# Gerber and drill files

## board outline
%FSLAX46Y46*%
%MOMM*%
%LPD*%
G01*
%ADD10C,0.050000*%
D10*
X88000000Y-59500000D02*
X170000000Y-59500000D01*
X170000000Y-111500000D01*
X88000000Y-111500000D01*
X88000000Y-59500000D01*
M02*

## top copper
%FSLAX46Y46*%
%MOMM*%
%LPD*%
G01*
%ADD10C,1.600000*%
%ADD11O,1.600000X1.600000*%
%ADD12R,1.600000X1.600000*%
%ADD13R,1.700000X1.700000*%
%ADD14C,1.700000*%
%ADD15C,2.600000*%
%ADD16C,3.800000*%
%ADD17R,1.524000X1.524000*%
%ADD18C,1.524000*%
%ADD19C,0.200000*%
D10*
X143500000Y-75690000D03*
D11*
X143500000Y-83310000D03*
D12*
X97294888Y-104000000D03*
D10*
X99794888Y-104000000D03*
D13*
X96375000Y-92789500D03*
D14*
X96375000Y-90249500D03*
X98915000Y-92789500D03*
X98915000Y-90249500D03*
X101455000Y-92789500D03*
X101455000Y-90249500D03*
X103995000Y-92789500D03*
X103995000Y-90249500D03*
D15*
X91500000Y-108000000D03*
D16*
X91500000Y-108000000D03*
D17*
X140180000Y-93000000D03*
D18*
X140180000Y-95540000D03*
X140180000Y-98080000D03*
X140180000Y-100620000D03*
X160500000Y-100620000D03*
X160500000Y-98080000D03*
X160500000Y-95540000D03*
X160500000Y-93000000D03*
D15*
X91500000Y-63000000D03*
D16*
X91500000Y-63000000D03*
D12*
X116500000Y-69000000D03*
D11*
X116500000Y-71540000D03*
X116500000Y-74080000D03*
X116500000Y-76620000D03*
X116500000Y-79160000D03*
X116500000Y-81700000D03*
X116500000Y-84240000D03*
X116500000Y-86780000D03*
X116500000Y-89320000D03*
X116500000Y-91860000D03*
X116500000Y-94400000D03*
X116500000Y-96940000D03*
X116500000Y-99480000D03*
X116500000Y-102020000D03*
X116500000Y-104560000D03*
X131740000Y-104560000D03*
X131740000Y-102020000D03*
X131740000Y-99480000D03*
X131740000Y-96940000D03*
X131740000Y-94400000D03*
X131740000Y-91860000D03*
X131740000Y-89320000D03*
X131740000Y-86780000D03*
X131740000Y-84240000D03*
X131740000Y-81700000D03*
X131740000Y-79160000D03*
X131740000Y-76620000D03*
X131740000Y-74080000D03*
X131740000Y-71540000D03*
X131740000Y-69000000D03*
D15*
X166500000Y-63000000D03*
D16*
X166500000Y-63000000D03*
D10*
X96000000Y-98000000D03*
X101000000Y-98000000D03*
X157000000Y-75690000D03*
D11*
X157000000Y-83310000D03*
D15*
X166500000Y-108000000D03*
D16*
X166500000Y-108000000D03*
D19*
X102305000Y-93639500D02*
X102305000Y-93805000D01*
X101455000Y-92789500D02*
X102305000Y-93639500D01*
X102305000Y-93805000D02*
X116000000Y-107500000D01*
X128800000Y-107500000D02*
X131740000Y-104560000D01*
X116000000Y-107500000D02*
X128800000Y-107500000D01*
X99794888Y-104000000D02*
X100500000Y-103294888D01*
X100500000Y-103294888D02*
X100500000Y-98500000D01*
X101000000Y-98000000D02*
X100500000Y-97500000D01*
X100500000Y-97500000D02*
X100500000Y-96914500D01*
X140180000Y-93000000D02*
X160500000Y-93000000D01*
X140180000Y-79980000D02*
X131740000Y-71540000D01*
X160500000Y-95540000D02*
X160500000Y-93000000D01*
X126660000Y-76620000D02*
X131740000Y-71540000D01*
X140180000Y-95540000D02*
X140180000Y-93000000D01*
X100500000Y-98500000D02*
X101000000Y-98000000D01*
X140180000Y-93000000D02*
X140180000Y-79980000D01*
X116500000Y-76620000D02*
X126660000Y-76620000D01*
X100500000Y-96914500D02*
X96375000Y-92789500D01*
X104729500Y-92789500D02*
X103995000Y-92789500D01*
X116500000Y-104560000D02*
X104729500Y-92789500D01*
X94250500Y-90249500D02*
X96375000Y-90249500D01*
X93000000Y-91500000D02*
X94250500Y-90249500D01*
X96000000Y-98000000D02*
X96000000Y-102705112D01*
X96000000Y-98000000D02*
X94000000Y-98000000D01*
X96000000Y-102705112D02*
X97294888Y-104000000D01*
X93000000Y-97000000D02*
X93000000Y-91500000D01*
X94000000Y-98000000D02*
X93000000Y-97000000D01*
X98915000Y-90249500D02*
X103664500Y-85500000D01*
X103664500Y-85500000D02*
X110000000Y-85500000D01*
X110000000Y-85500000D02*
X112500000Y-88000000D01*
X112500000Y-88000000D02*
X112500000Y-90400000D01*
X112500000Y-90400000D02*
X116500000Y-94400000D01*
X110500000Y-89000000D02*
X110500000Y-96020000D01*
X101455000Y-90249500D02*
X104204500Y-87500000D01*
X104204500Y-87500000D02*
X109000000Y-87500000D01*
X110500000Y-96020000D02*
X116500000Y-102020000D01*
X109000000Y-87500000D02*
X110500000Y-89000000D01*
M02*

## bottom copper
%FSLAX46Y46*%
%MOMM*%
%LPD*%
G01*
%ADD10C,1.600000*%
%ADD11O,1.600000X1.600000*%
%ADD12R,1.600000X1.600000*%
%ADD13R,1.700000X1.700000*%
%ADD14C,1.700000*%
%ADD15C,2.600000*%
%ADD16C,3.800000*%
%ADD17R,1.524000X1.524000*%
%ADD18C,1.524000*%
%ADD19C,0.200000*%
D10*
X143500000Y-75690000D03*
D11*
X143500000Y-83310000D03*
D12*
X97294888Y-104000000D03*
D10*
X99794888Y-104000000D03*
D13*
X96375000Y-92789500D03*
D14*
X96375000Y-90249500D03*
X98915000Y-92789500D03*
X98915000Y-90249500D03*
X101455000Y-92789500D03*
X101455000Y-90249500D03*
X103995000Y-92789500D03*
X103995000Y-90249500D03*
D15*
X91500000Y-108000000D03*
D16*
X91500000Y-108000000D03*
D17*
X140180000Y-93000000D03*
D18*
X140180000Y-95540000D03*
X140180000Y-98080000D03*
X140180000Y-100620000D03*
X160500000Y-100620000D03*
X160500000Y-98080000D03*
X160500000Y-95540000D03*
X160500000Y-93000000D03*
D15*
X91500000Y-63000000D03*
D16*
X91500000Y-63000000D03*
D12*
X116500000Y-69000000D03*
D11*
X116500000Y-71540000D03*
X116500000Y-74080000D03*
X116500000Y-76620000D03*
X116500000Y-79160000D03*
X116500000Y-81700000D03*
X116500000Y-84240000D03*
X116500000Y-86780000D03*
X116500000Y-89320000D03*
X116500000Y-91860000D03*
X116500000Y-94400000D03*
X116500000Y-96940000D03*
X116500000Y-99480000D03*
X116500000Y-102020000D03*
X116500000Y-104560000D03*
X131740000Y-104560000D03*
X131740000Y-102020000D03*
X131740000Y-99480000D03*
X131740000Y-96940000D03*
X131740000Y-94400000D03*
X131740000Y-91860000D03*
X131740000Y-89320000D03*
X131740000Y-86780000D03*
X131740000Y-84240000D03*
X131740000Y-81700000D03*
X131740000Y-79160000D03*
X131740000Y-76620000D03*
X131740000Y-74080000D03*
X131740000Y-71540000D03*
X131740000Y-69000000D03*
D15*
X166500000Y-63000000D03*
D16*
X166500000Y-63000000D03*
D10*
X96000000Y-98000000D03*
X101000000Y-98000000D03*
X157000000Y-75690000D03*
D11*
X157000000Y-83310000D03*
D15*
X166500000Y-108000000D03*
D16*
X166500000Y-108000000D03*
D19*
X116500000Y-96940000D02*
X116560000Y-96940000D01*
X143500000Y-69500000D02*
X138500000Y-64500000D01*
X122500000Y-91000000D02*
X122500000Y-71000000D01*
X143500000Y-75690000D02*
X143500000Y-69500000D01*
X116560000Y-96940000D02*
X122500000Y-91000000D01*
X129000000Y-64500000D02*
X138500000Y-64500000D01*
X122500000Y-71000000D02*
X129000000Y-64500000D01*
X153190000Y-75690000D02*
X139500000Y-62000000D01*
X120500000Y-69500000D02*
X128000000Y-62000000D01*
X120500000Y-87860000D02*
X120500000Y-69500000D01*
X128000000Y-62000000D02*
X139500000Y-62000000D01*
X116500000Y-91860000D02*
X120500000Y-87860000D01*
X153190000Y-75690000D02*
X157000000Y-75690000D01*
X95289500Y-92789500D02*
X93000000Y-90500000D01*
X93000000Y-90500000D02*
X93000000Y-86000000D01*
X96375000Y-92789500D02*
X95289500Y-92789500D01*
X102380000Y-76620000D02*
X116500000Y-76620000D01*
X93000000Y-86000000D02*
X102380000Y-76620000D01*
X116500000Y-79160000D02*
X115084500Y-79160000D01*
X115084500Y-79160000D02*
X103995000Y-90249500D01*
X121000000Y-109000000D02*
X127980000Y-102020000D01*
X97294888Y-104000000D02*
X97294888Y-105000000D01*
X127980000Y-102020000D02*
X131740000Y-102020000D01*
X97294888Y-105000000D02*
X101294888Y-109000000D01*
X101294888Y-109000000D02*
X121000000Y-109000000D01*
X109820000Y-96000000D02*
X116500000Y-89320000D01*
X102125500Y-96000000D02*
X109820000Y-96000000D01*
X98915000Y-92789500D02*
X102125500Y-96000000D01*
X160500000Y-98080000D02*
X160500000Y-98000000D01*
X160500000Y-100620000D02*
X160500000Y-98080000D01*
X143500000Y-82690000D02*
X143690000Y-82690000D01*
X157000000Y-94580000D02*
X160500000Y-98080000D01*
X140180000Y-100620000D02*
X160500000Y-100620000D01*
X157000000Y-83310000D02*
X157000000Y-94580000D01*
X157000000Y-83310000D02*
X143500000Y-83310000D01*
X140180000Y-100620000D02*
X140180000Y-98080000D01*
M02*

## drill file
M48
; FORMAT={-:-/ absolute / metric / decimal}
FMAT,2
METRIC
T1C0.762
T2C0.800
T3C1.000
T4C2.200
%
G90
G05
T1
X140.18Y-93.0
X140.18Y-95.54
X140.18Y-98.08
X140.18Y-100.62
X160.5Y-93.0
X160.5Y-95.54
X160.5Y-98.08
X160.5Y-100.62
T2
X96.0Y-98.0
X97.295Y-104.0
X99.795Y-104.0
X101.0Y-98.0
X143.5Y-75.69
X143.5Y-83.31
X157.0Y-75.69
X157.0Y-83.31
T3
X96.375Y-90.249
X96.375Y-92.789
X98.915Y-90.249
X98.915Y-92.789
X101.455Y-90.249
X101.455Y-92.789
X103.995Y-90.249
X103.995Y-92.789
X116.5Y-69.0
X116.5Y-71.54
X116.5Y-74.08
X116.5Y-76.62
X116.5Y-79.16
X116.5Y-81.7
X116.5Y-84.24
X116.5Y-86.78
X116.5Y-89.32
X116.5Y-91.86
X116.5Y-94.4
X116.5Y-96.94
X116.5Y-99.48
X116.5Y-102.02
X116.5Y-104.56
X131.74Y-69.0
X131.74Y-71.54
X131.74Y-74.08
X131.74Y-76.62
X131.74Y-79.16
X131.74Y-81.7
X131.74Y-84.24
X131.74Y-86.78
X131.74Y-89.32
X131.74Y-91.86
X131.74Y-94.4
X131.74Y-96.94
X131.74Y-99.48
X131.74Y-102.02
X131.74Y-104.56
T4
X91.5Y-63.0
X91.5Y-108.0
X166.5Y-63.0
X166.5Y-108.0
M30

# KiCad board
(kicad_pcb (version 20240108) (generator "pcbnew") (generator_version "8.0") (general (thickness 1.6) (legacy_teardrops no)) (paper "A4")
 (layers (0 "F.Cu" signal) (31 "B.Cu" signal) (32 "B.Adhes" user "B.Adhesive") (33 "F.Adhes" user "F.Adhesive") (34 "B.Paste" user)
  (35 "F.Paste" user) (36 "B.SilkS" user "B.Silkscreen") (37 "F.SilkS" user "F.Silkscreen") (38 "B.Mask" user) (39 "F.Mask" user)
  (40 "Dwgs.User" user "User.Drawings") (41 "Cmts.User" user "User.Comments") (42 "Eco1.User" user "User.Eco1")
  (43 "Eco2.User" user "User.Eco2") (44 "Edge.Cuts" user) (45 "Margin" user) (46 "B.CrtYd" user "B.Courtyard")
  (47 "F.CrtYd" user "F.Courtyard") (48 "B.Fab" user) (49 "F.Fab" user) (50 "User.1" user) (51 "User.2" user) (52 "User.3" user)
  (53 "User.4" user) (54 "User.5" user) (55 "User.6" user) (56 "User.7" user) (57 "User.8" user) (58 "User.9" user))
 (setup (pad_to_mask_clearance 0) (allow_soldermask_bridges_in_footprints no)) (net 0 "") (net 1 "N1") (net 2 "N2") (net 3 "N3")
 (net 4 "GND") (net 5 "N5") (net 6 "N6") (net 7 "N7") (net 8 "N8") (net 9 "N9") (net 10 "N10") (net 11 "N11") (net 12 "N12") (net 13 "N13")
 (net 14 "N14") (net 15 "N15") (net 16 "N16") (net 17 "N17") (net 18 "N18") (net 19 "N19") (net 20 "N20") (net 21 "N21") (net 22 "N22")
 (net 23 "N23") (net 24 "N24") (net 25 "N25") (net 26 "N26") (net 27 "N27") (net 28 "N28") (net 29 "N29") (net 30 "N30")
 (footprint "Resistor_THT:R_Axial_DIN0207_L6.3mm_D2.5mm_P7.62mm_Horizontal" (layer "F.Cu") (at 143.5 75.69 -90)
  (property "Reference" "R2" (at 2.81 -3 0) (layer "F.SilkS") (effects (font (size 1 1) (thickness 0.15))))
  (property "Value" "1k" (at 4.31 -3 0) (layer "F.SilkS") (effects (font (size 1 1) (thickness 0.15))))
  (pad "1" thru_hole circle (at 0 0 270) (size 1.6 1.6) (drill 0.8) (layers "*.Cu" "*.Mask") (remove_unused_layers no) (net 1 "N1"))
  (pad "2" thru_hole oval (at 7.62 0 270) (size 1.6 1.6) (drill 0.8) (layers "*.Cu" "*.Mask") (remove_unused_layers no) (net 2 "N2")))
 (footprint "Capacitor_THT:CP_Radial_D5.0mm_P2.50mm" (layer "F.Cu") (at 97.294888 104)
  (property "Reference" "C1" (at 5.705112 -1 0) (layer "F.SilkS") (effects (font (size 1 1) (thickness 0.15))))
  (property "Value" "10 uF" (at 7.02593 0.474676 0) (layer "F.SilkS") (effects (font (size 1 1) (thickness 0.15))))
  (pad "1" thru_hole rect (at 0 0) (size 1.6 1.6) (drill 0.8) (layers "*.Cu" "*.Mask") (remove_unused_layers no) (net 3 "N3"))
  (pad "2" thru_hole circle (at 2.5 0) (size 1.6 1.6) (drill 0.8) (layers "*.Cu" "*.Mask") (remove_unused_layers no) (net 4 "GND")))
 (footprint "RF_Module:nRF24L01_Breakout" (layer "F.Cu") (at 96.375 92.7895 90)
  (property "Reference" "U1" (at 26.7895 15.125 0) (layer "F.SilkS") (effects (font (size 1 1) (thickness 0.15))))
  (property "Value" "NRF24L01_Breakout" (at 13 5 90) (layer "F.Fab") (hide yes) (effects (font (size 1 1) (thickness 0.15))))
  (pad "1" thru_hole rect (at 0 0 90) (size 1.7 1.7) (drill 1) (layers "*.Cu" "*.Mask") (remove_unused_layers no) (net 4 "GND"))
  (pad "2" thru_hole circle (at 2.54 0 90) (size 1.7 1.7) (drill 1) (layers "*.Cu" "*.Mask") (remove_unused_layers no) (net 3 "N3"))
  (pad "3" thru_hole circle (at 0 2.54 90) (size 1.7 1.7) (drill 1) (layers "*.Cu" "*.Mask") (remove_unused_layers no) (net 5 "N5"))
  (pad "4" thru_hole circle (at 2.54 2.54 90) (size 1.7 1.7) (drill 1) (layers "*.Cu" "*.Mask") (remove_unused_layers no) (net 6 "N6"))
  (pad "5" thru_hole circle (at 0 5.08 90) (size 1.7 1.7) (drill 1) (layers "*.Cu" "*.Mask") (remove_unused_layers no) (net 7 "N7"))
  (pad "6" thru_hole circle (at 2.54 5.08 90) (size 1.7 1.7) (drill 1) (layers "*.Cu" "*.Mask") (remove_unused_layers no) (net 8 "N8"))
  (pad "7" thru_hole circle (at 0 7.62 90) (size 1.7 1.7) (drill 1) (layers "*.Cu" "*.Mask") (remove_unused_layers no) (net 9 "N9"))
  (pad "8" thru_hole circle (at 2.54 7.62 90) (size 1.7 1.7) (drill 1) (layers "*.Cu" "*.Mask") (remove_unused_layers no) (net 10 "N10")))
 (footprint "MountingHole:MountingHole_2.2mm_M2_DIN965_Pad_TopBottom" (layer "F.Cu") (at 91.5 108)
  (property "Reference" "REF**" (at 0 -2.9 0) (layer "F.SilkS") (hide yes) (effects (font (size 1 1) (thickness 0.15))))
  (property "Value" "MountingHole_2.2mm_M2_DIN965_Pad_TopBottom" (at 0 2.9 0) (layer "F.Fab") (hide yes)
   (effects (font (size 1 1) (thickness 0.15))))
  (pad "1" thru_hole circle (at 0 0) (size 2.6 2.6) (drill 2.2) (layers "*.Cu" "*.Mask") (remove_unused_layers no))
  (pad "1" connect circle (at 0 0) (size 3.8 3.8) (layers "F.Cu" "F.Mask"))
  (pad "1" connect circle (at 0 0) (size 3.8 3.8) (layers "B.Cu" "B.Mask")))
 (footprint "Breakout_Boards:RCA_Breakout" (layer "F.Cu") (at 150.38 100.5)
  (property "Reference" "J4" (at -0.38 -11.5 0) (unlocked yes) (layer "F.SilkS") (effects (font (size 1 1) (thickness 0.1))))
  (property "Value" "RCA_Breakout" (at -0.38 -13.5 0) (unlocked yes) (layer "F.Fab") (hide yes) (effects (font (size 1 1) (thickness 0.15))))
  (pad "1" thru_hole rect (at -10.2 -7.5) (size 1.524 1.524) (drill 0.762) (layers "*.Cu" "*.Mask") (remove_unused_layers no) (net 4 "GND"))
  (pad "2" thru_hole circle (at -10.2 -4.96) (size 1.524 1.524) (drill 0.762) (layers "*.Cu" "*.Mask") (remove_unused_layers no)
   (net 4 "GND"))
  (pad "3" thru_hole circle (at -10.2 -2.42) (size 1.524 1.524) (drill 0.762) (layers "*.Cu" "*.Mask") (remove_unused_layers no)
   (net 2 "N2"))
  (pad "4" thru_hole circle (at -10.2 0.12) (size 1.524 1.524) (drill 0.762) (layers "*.Cu" "*.Mask") (remove_unused_layers no) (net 2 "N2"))
  (pad "5" thru_hole circle (at 10.12 0.12) (size 1.524 1.524) (drill 0.762) (layers "*.Cu" "*.Mask") (remove_unused_layers no) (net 2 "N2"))
  (pad "6" thru_hole circle (at 10.12 -2.42) (size 1.524 1.524) (drill 0.762) (layers "*.Cu" "*.Mask") (remove_unused_layers no)
   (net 2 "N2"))
  (pad "7" thru_hole circle (at 10.12 -4.96) (size 1.524 1.524) (drill 0.762) (layers "*.Cu" "*.Mask") (remove_unused_layers no)
   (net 4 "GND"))
  (pad "8" thru_hole circle (at 10.12 -7.5) (size 1.524 1.524) (drill 0.762) (layers "*.Cu" "*.Mask") (remove_unused_layers no)
   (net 4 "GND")))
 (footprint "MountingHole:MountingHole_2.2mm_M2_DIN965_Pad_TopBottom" (layer "F.Cu") (at 91.5 63)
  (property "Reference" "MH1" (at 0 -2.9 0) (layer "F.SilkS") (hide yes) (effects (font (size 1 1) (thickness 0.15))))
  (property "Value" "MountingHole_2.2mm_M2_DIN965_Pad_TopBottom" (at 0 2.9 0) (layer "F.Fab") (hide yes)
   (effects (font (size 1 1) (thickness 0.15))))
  (pad "1" thru_hole circle (at 0 0) (size 2.6 2.6) (drill 2.2) (layers "*.Cu" "*.Mask") (remove_unused_layers no))
  (pad "1" connect circle (at 0 0) (size 3.8 3.8) (layers "F.Cu" "F.Mask"))
  (pad "1" connect circle (at 0 0) (size 3.8 3.8) (layers "B.Cu" "B.Mask")))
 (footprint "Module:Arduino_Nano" (layer "F.Cu") (at 116.5 69)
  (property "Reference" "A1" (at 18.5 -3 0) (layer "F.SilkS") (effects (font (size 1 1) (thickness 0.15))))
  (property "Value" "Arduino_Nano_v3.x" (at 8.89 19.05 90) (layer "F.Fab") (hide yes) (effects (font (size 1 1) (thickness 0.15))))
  (pad "1" thru_hole rect (at 0 0) (size 1.6 1.6) (drill 1) (layers "*.Cu" "*.Mask") (remove_unused_layers no) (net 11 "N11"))
  (pad "2" thru_hole oval (at 0 2.54) (size 1.6 1.6) (drill 1) (layers "*.Cu" "*.Mask") (remove_unused_layers no) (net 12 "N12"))
  (pad "3" thru_hole oval (at 0 5.08) (size 1.6 1.6) (drill 1) (layers "*.Cu" "*.Mask") (remove_unused_layers no) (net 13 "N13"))
  (pad "4" thru_hole oval (at 0 7.62) (size 1.6 1.6) (drill 1) (layers "*.Cu" "*.Mask") (remove_unused_layers no) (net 4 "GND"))
  (pad "5" thru_hole oval (at 0 10.16) (size 1.6 1.6) (drill 1) (layers "*.Cu" "*.Mask") (remove_unused_layers no) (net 10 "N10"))
  (pad "6" thru_hole oval (at 0 12.7) (size 1.6 1.6) (drill 1) (layers "*.Cu" "*.Mask") (remove_unused_layers no) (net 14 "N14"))
  (pad "7" thru_hole oval (at 0 15.24) (size 1.6 1.6) (drill 1) (layers "*.Cu" "*.Mask") (remove_unused_layers no) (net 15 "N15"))
  (pad "8" thru_hole oval (at 0 17.78) (size 1.6 1.6) (drill 1) (layers "*.Cu" "*.Mask") (remove_unused_layers no) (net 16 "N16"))
  (pad "9" thru_hole oval (at 0 20.32) (size 1.6 1.6) (drill 1) (layers "*.Cu" "*.Mask") (remove_unused_layers no) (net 5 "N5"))
  (pad "10" thru_hole oval (at 0 22.86) (size 1.6 1.6) (drill 1) (layers "*.Cu" "*.Mask") (remove_unused_layers no) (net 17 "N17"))
  (pad "11" thru_hole oval (at 0 25.4) (size 1.6 1.6) (drill 1) (layers "*.Cu" "*.Mask") (remove_unused_layers no) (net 6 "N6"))
  (pad "12" thru_hole oval (at 0 27.94) (size 1.6 1.6) (drill 1) (layers "*.Cu" "*.Mask") (remove_unused_layers no) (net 1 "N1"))
  (pad "13" thru_hole oval (at 0 30.48) (size 1.6 1.6) (drill 1) (layers "*.Cu" "*.Mask") (remove_unused_layers no) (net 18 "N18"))
  (pad "14" thru_hole oval (at 0 33.02) (size 1.6 1.6) (drill 1) (layers "*.Cu" "*.Mask") (remove_unused_layers no) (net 8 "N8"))
  (pad "15" thru_hole oval (at 0 35.56) (size 1.6 1.6) (drill 1) (layers "*.Cu" "*.Mask") (remove_unused_layers no) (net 9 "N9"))
  (pad "16" thru_hole oval (at 15.24 35.56) (size 1.6 1.6) (drill 1) (layers "*.Cu" "*.Mask") (remove_unused_layers no) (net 7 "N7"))
  (pad "17" thru_hole oval (at 15.24 33.02) (size 1.6 1.6) (drill 1) (layers "*.Cu" "*.Mask") (remove_unused_layers no) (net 3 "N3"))
  (pad "18" thru_hole oval (at 15.24 30.48) (size 1.6 1.6) (drill 1) (layers "*.Cu" "*.Mask") (remove_unused_layers no) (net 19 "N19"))
  (pad "19" thru_hole oval (at 15.24 27.94) (size 1.6 1.6) (drill 1) (layers "*.Cu" "*.Mask") (remove_unused_layers no) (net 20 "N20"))
  (pad "20" thru_hole oval (at 15.24 25.4) (size 1.6 1.6) (drill 1) (layers "*.Cu" "*.Mask") (remove_unused_layers no) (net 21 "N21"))
  (pad "21" thru_hole oval (at 15.24 22.86) (size 1.6 1.6) (drill 1) (layers "*.Cu" "*.Mask") (remove_unused_layers no) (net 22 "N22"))
  (pad "22" thru_hole oval (at 15.24 20.32) (size 1.6 1.6) (drill 1) (layers "*.Cu" "*.Mask") (remove_unused_layers no) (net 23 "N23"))
  (pad "23" thru_hole oval (at 15.24 17.78) (size 1.6 1.6) (drill 1) (layers "*.Cu" "*.Mask") (remove_unused_layers no) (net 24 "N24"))
  (pad "24" thru_hole oval (at 15.24 15.24) (size 1.6 1.6) (drill 1) (layers "*.Cu" "*.Mask") (remove_unused_layers no) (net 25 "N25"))
  (pad "25" thru_hole oval (at 15.24 12.7) (size 1.6 1.6) (drill 1) (layers "*.Cu" "*.Mask") (remove_unused_layers no) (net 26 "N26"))
  (pad "26" thru_hole oval (at 15.24 10.16) (size 1.6 1.6) (drill 1) (layers "*.Cu" "*.Mask") (remove_unused_layers no) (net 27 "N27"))
  (pad "27" thru_hole oval (at 15.24 7.62) (size 1.6 1.6) (drill 1) (layers "*.Cu" "*.Mask") (remove_unused_layers no) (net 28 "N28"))
  (pad "28" thru_hole oval (at 15.24 5.08) (size 1.6 1.6) (drill 1) (layers "*.Cu" "*.Mask") (remove_unused_layers no) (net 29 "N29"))
  (pad "29" thru_hole oval (at 15.24 2.54) (size 1.6 1.6) (drill 1) (layers "*.Cu" "*.Mask") (remove_unused_layers no) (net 4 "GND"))
  (pad "30" thru_hole oval (at 15.24 0) (size 1.6 1.6) (drill 1) (layers "*.Cu" "*.Mask") (remove_unused_layers no) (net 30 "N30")))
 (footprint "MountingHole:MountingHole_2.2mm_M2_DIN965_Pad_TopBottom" (layer "F.Cu") (at 166.5 63)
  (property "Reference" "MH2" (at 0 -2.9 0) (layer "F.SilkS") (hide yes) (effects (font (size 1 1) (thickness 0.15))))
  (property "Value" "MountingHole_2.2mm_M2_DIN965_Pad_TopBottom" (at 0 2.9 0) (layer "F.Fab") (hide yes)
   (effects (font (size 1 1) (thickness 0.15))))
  (pad "1" thru_hole circle (at 0 0) (size 2.6 2.6) (drill 2.2) (layers "*.Cu" "*.Mask") (remove_unused_layers no))
  (pad "1" connect circle (at 0 0) (size 3.8 3.8) (layers "F.Cu" "F.Mask"))
  (pad "1" connect circle (at 0 0) (size 3.8 3.8) (layers "B.Cu" "B.Mask")))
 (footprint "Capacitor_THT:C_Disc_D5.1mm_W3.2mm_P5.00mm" (layer "F.Cu") (at 96 98)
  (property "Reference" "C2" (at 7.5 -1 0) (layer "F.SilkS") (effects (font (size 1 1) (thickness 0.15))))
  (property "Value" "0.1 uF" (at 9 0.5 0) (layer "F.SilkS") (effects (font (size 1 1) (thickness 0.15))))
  (pad "1" thru_hole circle (at 0 0) (size 1.6 1.6) (drill 0.8) (layers "*.Cu" "*.Mask") (remove_unused_layers no) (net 3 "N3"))
  (pad "2" thru_hole circle (at 5 0) (size 1.6 1.6) (drill 0.8) (layers "*.Cu" "*.Mask") (remove_unused_layers no) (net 4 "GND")))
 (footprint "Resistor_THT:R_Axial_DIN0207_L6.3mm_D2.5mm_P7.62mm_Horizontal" (layer "F.Cu") (at 157 75.69 -90)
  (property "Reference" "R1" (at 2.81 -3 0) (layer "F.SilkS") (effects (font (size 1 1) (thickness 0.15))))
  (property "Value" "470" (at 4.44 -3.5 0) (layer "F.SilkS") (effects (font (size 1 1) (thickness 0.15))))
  (pad "1" thru_hole circle (at 0 0 270) (size 1.6 1.6) (drill 0.8) (layers "*.Cu" "*.Mask") (remove_unused_layers no) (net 17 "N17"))
  (pad "2" thru_hole oval (at 7.62 0 270) (size 1.6 1.6) (drill 0.8) (layers "*.Cu" "*.Mask") (remove_unused_layers no) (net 2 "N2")))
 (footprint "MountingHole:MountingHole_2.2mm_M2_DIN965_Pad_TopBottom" (layer "F.Cu") (at 166.5 108)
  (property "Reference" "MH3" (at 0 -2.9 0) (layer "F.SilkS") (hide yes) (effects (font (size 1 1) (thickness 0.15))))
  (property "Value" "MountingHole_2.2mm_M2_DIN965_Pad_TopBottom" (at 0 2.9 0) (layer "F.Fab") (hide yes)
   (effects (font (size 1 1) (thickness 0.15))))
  (pad "1" thru_hole circle (at 0 0) (size 2.6 2.6) (drill 2.2) (layers "*.Cu" "*.Mask") (remove_unused_layers no))
  (pad "1" connect circle (at 0 0) (size 3.8 3.8) (layers "F.Cu" "F.Mask"))
  (pad "1" connect circle (at 0 0) (size 3.8 3.8) (layers "B.Cu" "B.Mask")))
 (gr_rect (start 88 59.5) (end 170 111.5) (stroke (width 0.05) (type default)) (fill none) (layer "Edge.Cuts"))
 (segment (start 102.305 93.6395) (end 102.305 93.805) (width 0.2) (layer "F.Cu") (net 7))
 (segment (start 101.455 92.7895) (end 102.305 93.6395) (width 0.2) (layer "F.Cu") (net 7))
 (segment (start 102.305 93.805) (end 116 107.5) (width 0.2) (layer "F.Cu") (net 7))
 (segment (start 128.8 107.5) (end 131.74 104.56) (width 0.2) (layer "F.Cu") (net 7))
 (segment (start 116 107.5) (end 128.8 107.5) (width 0.2) (layer "F.Cu") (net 7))
 (segment (start 116.5 96.94) (end 116.56 96.94) (width 0.2) (layer "B.Cu") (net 1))
 (segment (start 143.5 69.5) (end 138.5 64.5) (width 0.2) (layer "B.Cu") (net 1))
 (segment (start 122.5 91) (end 122.5 71) (width 0.2) (layer "B.Cu") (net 1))
 (segment (start 143.5 75.69) (end 143.5 69.5) (width 0.2) (layer "B.Cu") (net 1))
 (segment (start 116.56 96.94) (end 122.5 91) (width 0.2) (layer "B.Cu") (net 1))
 (segment (start 129 64.5) (end 138.5 64.5) (width 0.2) (layer "B.Cu") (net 1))
 (segment (start 122.5 71) (end 129 64.5) (width 0.2) (layer "B.Cu") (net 1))
 (segment (start 153.19 75.69) (end 139.5 62) (width 0.2) (layer "B.Cu") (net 17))
 (segment (start 120.5 69.5) (end 128 62) (width 0.2) (layer "B.Cu") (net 17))
 (segment (start 120.5 87.86) (end 120.5 69.5) (width 0.2) (layer "B.Cu") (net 17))
 (segment (start 128 62) (end 139.5 62) (width 0.2) (layer "B.Cu") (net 17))
 (segment (start 116.5 91.86) (end 120.5 87.86) (width 0.2) (layer "B.Cu") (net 17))
 (segment (start 153.19 75.69) (end 157 75.69) (width 0.2) (layer "B.Cu") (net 17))
 (segment (start 99.794888 104) (end 100.5 103.294888) (width 0.2) (layer "F.Cu") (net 4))
 (segment (start 100.5 103.294888) (end 100.5 98.5) (width 0.2) (layer "F.Cu") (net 4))
 (segment (start 101 98) (end 100.5 97.5) (width 0.2) (layer "F.Cu") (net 4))
 (segment (start 100.5 97.5) (end 100.5 96.9145) (width 0.2) (layer "F.Cu") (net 4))
 (segment (start 140.18 93) (end 160.5 93) (width 0.2) (layer "F.Cu") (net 4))
 (segment (start 140.18 79.98) (end 131.74 71.54) (width 0.2) (layer "F.Cu") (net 4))
 (segment (start 160.5 95.54) (end 160.5 93) (width 0.2) (layer "F.Cu") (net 4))
 (segment (start 126.66 76.62) (end 131.74 71.54) (width 0.2) (layer "F.Cu") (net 4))
 (segment (start 140.18 95.54) (end 140.18 93) (width 0.2) (layer "F.Cu") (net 4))
 (segment (start 100.5 98.5) (end 101 98) (width 0.2) (layer "F.Cu") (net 4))
 (segment (start 140.18 93) (end 140.18 79.98) (width 0.2) (layer "F.Cu") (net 4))
 (segment (start 116.5 76.62) (end 126.66 76.62) (width 0.2) (layer "F.Cu") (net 4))
 (segment (start 100.5 96.9145) (end 96.375 92.7895) (width 0.2) (layer "F.Cu") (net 4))
 (segment (start 95.2895 92.7895) (end 93 90.5) (width 0.2) (layer "B.Cu") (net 4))
 (segment (start 93 90.5) (end 93 86) (width 0.2) (layer "B.Cu") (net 4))
 (segment (start 96.375 92.7895) (end 95.2895 92.7895) (width 0.2) (layer "B.Cu") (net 4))
 (segment (start 102.38 76.62) (end 116.5 76.62) (width 0.2) (layer "B.Cu") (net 4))
 (segment (start 93 86) (end 102.38 76.62) (width 0.2) (layer "B.Cu") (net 4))
 (segment (start 104.7295 92.7895) (end 103.995 92.7895) (width 0.2) (layer "F.Cu") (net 9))
 (segment (start 116.5 104.56) (end 104.7295 92.7895) (width 0.2) (layer "F.Cu") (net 9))
 (segment (start 116.5 79.16) (end 115.0845 79.16) (width 0.2) (layer "B.Cu") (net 10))
 (segment (start 115.0845 79.16) (end 103.995 90.2495) (width 0.2) (layer "B.Cu") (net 10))
 (segment (start 94.2505 90.2495) (end 96.375 90.2495) (width 0.2) (layer "F.Cu") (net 3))
 (segment (start 93 91.5) (end 94.2505 90.2495) (width 0.2) (layer "F.Cu") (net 3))
 (segment (start 96 98) (end 96 102.705112) (width 0.2) (layer "F.Cu") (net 3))
 (segment (start 96 98) (end 94 98) (width 0.2) (layer "F.Cu") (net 3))
 (segment (start 96 102.705112) (end 97.294888 104) (width 0.2) (layer "F.Cu") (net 3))
 (segment (start 93 97) (end 93 91.5) (width 0.2) (layer "F.Cu") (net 3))
 (segment (start 94 98) (end 93 97) (width 0.2) (layer "F.Cu") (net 3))
 (segment (start 121 109) (end 127.98 102.02) (width 0.2) (layer "B.Cu") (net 3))
 (segment (start 97.294888 104) (end 97.294888 105) (width 0.2) (layer "B.Cu") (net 3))
 (segment (start 127.98 102.02) (end 131.74 102.02) (width 0.2) (layer "B.Cu") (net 3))
 (segment (start 97.294888 105) (end 101.294888 109) (width 0.2) (layer "B.Cu") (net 3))
 (segment (start 101.294888 109) (end 121 109) (width 0.2) (layer "B.Cu") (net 3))
 (segment (start 98.915 90.2495) (end 103.6645 85.5) (width 0.2) (layer "F.Cu") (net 6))
 (segment (start 103.6645 85.5) (end 110 85.5) (width 0.2) (layer "F.Cu") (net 6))
 (segment (start 110 85.5) (end 112.5 88) (width 0.2) (layer "F.Cu") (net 6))
 (segment (start 112.5 88) (end 112.5 90.4) (width 0.2) (layer "F.Cu") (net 6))
 (segment (start 112.5 90.4) (end 116.5 94.4) (width 0.2) (layer "F.Cu") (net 6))
 (segment (start 110.5 89) (end 110.5 96.02) (width 0.2) (layer "F.Cu") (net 8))
 (segment (start 101.455 90.2495) (end 104.2045 87.5) (width 0.2) (layer "F.Cu") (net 8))
 (segment (start 104.2045 87.5) (end 109 87.5) (width 0.2) (layer "F.Cu") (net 8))
 (segment (start 110.5 96.02) (end 116.5 102.02) (width 0.2) (layer "F.Cu") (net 8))
 (segment (start 109 87.5) (end 110.5 89) (width 0.2) (layer "F.Cu") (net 8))
 (segment (start 109.82 96) (end 116.5 89.32) (width 0.2) (layer "B.Cu") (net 5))
 (segment (start 102.1255 96) (end 109.82 96) (width 0.2) (layer "B.Cu") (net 5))
 (segment (start 98.915 92.7895) (end 102.1255 96) (width 0.2) (layer "B.Cu") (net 5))
 (segment (start 160.5 98.08) (end 160.5 98) (width 0.2) (layer "B.Cu") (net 2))
 (segment (start 160.5 100.62) (end 160.5 98.08) (width 0.2) (layer "B.Cu") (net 2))
 (segment (start 143.5 82.69) (end 143.69 82.69) (width 0.2) (layer "B.Cu") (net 2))
 (segment (start 157 94.58) (end 160.5 98.08) (width 0.2) (layer "B.Cu") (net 2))
 (segment (start 140.18 100.62) (end 160.5 100.62) (width 0.2) (layer "B.Cu") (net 2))
 (segment (start 157 83.31) (end 157 94.58) (width 0.2) (layer "B.Cu") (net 2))
 (segment (start 157 83.31) (end 143.5 83.31) (width 0.2) (layer "B.Cu") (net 2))
 (segment (start 140.18 100.62) (end 140.18 98.08) (width 0.2) (layer "B.Cu") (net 2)))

